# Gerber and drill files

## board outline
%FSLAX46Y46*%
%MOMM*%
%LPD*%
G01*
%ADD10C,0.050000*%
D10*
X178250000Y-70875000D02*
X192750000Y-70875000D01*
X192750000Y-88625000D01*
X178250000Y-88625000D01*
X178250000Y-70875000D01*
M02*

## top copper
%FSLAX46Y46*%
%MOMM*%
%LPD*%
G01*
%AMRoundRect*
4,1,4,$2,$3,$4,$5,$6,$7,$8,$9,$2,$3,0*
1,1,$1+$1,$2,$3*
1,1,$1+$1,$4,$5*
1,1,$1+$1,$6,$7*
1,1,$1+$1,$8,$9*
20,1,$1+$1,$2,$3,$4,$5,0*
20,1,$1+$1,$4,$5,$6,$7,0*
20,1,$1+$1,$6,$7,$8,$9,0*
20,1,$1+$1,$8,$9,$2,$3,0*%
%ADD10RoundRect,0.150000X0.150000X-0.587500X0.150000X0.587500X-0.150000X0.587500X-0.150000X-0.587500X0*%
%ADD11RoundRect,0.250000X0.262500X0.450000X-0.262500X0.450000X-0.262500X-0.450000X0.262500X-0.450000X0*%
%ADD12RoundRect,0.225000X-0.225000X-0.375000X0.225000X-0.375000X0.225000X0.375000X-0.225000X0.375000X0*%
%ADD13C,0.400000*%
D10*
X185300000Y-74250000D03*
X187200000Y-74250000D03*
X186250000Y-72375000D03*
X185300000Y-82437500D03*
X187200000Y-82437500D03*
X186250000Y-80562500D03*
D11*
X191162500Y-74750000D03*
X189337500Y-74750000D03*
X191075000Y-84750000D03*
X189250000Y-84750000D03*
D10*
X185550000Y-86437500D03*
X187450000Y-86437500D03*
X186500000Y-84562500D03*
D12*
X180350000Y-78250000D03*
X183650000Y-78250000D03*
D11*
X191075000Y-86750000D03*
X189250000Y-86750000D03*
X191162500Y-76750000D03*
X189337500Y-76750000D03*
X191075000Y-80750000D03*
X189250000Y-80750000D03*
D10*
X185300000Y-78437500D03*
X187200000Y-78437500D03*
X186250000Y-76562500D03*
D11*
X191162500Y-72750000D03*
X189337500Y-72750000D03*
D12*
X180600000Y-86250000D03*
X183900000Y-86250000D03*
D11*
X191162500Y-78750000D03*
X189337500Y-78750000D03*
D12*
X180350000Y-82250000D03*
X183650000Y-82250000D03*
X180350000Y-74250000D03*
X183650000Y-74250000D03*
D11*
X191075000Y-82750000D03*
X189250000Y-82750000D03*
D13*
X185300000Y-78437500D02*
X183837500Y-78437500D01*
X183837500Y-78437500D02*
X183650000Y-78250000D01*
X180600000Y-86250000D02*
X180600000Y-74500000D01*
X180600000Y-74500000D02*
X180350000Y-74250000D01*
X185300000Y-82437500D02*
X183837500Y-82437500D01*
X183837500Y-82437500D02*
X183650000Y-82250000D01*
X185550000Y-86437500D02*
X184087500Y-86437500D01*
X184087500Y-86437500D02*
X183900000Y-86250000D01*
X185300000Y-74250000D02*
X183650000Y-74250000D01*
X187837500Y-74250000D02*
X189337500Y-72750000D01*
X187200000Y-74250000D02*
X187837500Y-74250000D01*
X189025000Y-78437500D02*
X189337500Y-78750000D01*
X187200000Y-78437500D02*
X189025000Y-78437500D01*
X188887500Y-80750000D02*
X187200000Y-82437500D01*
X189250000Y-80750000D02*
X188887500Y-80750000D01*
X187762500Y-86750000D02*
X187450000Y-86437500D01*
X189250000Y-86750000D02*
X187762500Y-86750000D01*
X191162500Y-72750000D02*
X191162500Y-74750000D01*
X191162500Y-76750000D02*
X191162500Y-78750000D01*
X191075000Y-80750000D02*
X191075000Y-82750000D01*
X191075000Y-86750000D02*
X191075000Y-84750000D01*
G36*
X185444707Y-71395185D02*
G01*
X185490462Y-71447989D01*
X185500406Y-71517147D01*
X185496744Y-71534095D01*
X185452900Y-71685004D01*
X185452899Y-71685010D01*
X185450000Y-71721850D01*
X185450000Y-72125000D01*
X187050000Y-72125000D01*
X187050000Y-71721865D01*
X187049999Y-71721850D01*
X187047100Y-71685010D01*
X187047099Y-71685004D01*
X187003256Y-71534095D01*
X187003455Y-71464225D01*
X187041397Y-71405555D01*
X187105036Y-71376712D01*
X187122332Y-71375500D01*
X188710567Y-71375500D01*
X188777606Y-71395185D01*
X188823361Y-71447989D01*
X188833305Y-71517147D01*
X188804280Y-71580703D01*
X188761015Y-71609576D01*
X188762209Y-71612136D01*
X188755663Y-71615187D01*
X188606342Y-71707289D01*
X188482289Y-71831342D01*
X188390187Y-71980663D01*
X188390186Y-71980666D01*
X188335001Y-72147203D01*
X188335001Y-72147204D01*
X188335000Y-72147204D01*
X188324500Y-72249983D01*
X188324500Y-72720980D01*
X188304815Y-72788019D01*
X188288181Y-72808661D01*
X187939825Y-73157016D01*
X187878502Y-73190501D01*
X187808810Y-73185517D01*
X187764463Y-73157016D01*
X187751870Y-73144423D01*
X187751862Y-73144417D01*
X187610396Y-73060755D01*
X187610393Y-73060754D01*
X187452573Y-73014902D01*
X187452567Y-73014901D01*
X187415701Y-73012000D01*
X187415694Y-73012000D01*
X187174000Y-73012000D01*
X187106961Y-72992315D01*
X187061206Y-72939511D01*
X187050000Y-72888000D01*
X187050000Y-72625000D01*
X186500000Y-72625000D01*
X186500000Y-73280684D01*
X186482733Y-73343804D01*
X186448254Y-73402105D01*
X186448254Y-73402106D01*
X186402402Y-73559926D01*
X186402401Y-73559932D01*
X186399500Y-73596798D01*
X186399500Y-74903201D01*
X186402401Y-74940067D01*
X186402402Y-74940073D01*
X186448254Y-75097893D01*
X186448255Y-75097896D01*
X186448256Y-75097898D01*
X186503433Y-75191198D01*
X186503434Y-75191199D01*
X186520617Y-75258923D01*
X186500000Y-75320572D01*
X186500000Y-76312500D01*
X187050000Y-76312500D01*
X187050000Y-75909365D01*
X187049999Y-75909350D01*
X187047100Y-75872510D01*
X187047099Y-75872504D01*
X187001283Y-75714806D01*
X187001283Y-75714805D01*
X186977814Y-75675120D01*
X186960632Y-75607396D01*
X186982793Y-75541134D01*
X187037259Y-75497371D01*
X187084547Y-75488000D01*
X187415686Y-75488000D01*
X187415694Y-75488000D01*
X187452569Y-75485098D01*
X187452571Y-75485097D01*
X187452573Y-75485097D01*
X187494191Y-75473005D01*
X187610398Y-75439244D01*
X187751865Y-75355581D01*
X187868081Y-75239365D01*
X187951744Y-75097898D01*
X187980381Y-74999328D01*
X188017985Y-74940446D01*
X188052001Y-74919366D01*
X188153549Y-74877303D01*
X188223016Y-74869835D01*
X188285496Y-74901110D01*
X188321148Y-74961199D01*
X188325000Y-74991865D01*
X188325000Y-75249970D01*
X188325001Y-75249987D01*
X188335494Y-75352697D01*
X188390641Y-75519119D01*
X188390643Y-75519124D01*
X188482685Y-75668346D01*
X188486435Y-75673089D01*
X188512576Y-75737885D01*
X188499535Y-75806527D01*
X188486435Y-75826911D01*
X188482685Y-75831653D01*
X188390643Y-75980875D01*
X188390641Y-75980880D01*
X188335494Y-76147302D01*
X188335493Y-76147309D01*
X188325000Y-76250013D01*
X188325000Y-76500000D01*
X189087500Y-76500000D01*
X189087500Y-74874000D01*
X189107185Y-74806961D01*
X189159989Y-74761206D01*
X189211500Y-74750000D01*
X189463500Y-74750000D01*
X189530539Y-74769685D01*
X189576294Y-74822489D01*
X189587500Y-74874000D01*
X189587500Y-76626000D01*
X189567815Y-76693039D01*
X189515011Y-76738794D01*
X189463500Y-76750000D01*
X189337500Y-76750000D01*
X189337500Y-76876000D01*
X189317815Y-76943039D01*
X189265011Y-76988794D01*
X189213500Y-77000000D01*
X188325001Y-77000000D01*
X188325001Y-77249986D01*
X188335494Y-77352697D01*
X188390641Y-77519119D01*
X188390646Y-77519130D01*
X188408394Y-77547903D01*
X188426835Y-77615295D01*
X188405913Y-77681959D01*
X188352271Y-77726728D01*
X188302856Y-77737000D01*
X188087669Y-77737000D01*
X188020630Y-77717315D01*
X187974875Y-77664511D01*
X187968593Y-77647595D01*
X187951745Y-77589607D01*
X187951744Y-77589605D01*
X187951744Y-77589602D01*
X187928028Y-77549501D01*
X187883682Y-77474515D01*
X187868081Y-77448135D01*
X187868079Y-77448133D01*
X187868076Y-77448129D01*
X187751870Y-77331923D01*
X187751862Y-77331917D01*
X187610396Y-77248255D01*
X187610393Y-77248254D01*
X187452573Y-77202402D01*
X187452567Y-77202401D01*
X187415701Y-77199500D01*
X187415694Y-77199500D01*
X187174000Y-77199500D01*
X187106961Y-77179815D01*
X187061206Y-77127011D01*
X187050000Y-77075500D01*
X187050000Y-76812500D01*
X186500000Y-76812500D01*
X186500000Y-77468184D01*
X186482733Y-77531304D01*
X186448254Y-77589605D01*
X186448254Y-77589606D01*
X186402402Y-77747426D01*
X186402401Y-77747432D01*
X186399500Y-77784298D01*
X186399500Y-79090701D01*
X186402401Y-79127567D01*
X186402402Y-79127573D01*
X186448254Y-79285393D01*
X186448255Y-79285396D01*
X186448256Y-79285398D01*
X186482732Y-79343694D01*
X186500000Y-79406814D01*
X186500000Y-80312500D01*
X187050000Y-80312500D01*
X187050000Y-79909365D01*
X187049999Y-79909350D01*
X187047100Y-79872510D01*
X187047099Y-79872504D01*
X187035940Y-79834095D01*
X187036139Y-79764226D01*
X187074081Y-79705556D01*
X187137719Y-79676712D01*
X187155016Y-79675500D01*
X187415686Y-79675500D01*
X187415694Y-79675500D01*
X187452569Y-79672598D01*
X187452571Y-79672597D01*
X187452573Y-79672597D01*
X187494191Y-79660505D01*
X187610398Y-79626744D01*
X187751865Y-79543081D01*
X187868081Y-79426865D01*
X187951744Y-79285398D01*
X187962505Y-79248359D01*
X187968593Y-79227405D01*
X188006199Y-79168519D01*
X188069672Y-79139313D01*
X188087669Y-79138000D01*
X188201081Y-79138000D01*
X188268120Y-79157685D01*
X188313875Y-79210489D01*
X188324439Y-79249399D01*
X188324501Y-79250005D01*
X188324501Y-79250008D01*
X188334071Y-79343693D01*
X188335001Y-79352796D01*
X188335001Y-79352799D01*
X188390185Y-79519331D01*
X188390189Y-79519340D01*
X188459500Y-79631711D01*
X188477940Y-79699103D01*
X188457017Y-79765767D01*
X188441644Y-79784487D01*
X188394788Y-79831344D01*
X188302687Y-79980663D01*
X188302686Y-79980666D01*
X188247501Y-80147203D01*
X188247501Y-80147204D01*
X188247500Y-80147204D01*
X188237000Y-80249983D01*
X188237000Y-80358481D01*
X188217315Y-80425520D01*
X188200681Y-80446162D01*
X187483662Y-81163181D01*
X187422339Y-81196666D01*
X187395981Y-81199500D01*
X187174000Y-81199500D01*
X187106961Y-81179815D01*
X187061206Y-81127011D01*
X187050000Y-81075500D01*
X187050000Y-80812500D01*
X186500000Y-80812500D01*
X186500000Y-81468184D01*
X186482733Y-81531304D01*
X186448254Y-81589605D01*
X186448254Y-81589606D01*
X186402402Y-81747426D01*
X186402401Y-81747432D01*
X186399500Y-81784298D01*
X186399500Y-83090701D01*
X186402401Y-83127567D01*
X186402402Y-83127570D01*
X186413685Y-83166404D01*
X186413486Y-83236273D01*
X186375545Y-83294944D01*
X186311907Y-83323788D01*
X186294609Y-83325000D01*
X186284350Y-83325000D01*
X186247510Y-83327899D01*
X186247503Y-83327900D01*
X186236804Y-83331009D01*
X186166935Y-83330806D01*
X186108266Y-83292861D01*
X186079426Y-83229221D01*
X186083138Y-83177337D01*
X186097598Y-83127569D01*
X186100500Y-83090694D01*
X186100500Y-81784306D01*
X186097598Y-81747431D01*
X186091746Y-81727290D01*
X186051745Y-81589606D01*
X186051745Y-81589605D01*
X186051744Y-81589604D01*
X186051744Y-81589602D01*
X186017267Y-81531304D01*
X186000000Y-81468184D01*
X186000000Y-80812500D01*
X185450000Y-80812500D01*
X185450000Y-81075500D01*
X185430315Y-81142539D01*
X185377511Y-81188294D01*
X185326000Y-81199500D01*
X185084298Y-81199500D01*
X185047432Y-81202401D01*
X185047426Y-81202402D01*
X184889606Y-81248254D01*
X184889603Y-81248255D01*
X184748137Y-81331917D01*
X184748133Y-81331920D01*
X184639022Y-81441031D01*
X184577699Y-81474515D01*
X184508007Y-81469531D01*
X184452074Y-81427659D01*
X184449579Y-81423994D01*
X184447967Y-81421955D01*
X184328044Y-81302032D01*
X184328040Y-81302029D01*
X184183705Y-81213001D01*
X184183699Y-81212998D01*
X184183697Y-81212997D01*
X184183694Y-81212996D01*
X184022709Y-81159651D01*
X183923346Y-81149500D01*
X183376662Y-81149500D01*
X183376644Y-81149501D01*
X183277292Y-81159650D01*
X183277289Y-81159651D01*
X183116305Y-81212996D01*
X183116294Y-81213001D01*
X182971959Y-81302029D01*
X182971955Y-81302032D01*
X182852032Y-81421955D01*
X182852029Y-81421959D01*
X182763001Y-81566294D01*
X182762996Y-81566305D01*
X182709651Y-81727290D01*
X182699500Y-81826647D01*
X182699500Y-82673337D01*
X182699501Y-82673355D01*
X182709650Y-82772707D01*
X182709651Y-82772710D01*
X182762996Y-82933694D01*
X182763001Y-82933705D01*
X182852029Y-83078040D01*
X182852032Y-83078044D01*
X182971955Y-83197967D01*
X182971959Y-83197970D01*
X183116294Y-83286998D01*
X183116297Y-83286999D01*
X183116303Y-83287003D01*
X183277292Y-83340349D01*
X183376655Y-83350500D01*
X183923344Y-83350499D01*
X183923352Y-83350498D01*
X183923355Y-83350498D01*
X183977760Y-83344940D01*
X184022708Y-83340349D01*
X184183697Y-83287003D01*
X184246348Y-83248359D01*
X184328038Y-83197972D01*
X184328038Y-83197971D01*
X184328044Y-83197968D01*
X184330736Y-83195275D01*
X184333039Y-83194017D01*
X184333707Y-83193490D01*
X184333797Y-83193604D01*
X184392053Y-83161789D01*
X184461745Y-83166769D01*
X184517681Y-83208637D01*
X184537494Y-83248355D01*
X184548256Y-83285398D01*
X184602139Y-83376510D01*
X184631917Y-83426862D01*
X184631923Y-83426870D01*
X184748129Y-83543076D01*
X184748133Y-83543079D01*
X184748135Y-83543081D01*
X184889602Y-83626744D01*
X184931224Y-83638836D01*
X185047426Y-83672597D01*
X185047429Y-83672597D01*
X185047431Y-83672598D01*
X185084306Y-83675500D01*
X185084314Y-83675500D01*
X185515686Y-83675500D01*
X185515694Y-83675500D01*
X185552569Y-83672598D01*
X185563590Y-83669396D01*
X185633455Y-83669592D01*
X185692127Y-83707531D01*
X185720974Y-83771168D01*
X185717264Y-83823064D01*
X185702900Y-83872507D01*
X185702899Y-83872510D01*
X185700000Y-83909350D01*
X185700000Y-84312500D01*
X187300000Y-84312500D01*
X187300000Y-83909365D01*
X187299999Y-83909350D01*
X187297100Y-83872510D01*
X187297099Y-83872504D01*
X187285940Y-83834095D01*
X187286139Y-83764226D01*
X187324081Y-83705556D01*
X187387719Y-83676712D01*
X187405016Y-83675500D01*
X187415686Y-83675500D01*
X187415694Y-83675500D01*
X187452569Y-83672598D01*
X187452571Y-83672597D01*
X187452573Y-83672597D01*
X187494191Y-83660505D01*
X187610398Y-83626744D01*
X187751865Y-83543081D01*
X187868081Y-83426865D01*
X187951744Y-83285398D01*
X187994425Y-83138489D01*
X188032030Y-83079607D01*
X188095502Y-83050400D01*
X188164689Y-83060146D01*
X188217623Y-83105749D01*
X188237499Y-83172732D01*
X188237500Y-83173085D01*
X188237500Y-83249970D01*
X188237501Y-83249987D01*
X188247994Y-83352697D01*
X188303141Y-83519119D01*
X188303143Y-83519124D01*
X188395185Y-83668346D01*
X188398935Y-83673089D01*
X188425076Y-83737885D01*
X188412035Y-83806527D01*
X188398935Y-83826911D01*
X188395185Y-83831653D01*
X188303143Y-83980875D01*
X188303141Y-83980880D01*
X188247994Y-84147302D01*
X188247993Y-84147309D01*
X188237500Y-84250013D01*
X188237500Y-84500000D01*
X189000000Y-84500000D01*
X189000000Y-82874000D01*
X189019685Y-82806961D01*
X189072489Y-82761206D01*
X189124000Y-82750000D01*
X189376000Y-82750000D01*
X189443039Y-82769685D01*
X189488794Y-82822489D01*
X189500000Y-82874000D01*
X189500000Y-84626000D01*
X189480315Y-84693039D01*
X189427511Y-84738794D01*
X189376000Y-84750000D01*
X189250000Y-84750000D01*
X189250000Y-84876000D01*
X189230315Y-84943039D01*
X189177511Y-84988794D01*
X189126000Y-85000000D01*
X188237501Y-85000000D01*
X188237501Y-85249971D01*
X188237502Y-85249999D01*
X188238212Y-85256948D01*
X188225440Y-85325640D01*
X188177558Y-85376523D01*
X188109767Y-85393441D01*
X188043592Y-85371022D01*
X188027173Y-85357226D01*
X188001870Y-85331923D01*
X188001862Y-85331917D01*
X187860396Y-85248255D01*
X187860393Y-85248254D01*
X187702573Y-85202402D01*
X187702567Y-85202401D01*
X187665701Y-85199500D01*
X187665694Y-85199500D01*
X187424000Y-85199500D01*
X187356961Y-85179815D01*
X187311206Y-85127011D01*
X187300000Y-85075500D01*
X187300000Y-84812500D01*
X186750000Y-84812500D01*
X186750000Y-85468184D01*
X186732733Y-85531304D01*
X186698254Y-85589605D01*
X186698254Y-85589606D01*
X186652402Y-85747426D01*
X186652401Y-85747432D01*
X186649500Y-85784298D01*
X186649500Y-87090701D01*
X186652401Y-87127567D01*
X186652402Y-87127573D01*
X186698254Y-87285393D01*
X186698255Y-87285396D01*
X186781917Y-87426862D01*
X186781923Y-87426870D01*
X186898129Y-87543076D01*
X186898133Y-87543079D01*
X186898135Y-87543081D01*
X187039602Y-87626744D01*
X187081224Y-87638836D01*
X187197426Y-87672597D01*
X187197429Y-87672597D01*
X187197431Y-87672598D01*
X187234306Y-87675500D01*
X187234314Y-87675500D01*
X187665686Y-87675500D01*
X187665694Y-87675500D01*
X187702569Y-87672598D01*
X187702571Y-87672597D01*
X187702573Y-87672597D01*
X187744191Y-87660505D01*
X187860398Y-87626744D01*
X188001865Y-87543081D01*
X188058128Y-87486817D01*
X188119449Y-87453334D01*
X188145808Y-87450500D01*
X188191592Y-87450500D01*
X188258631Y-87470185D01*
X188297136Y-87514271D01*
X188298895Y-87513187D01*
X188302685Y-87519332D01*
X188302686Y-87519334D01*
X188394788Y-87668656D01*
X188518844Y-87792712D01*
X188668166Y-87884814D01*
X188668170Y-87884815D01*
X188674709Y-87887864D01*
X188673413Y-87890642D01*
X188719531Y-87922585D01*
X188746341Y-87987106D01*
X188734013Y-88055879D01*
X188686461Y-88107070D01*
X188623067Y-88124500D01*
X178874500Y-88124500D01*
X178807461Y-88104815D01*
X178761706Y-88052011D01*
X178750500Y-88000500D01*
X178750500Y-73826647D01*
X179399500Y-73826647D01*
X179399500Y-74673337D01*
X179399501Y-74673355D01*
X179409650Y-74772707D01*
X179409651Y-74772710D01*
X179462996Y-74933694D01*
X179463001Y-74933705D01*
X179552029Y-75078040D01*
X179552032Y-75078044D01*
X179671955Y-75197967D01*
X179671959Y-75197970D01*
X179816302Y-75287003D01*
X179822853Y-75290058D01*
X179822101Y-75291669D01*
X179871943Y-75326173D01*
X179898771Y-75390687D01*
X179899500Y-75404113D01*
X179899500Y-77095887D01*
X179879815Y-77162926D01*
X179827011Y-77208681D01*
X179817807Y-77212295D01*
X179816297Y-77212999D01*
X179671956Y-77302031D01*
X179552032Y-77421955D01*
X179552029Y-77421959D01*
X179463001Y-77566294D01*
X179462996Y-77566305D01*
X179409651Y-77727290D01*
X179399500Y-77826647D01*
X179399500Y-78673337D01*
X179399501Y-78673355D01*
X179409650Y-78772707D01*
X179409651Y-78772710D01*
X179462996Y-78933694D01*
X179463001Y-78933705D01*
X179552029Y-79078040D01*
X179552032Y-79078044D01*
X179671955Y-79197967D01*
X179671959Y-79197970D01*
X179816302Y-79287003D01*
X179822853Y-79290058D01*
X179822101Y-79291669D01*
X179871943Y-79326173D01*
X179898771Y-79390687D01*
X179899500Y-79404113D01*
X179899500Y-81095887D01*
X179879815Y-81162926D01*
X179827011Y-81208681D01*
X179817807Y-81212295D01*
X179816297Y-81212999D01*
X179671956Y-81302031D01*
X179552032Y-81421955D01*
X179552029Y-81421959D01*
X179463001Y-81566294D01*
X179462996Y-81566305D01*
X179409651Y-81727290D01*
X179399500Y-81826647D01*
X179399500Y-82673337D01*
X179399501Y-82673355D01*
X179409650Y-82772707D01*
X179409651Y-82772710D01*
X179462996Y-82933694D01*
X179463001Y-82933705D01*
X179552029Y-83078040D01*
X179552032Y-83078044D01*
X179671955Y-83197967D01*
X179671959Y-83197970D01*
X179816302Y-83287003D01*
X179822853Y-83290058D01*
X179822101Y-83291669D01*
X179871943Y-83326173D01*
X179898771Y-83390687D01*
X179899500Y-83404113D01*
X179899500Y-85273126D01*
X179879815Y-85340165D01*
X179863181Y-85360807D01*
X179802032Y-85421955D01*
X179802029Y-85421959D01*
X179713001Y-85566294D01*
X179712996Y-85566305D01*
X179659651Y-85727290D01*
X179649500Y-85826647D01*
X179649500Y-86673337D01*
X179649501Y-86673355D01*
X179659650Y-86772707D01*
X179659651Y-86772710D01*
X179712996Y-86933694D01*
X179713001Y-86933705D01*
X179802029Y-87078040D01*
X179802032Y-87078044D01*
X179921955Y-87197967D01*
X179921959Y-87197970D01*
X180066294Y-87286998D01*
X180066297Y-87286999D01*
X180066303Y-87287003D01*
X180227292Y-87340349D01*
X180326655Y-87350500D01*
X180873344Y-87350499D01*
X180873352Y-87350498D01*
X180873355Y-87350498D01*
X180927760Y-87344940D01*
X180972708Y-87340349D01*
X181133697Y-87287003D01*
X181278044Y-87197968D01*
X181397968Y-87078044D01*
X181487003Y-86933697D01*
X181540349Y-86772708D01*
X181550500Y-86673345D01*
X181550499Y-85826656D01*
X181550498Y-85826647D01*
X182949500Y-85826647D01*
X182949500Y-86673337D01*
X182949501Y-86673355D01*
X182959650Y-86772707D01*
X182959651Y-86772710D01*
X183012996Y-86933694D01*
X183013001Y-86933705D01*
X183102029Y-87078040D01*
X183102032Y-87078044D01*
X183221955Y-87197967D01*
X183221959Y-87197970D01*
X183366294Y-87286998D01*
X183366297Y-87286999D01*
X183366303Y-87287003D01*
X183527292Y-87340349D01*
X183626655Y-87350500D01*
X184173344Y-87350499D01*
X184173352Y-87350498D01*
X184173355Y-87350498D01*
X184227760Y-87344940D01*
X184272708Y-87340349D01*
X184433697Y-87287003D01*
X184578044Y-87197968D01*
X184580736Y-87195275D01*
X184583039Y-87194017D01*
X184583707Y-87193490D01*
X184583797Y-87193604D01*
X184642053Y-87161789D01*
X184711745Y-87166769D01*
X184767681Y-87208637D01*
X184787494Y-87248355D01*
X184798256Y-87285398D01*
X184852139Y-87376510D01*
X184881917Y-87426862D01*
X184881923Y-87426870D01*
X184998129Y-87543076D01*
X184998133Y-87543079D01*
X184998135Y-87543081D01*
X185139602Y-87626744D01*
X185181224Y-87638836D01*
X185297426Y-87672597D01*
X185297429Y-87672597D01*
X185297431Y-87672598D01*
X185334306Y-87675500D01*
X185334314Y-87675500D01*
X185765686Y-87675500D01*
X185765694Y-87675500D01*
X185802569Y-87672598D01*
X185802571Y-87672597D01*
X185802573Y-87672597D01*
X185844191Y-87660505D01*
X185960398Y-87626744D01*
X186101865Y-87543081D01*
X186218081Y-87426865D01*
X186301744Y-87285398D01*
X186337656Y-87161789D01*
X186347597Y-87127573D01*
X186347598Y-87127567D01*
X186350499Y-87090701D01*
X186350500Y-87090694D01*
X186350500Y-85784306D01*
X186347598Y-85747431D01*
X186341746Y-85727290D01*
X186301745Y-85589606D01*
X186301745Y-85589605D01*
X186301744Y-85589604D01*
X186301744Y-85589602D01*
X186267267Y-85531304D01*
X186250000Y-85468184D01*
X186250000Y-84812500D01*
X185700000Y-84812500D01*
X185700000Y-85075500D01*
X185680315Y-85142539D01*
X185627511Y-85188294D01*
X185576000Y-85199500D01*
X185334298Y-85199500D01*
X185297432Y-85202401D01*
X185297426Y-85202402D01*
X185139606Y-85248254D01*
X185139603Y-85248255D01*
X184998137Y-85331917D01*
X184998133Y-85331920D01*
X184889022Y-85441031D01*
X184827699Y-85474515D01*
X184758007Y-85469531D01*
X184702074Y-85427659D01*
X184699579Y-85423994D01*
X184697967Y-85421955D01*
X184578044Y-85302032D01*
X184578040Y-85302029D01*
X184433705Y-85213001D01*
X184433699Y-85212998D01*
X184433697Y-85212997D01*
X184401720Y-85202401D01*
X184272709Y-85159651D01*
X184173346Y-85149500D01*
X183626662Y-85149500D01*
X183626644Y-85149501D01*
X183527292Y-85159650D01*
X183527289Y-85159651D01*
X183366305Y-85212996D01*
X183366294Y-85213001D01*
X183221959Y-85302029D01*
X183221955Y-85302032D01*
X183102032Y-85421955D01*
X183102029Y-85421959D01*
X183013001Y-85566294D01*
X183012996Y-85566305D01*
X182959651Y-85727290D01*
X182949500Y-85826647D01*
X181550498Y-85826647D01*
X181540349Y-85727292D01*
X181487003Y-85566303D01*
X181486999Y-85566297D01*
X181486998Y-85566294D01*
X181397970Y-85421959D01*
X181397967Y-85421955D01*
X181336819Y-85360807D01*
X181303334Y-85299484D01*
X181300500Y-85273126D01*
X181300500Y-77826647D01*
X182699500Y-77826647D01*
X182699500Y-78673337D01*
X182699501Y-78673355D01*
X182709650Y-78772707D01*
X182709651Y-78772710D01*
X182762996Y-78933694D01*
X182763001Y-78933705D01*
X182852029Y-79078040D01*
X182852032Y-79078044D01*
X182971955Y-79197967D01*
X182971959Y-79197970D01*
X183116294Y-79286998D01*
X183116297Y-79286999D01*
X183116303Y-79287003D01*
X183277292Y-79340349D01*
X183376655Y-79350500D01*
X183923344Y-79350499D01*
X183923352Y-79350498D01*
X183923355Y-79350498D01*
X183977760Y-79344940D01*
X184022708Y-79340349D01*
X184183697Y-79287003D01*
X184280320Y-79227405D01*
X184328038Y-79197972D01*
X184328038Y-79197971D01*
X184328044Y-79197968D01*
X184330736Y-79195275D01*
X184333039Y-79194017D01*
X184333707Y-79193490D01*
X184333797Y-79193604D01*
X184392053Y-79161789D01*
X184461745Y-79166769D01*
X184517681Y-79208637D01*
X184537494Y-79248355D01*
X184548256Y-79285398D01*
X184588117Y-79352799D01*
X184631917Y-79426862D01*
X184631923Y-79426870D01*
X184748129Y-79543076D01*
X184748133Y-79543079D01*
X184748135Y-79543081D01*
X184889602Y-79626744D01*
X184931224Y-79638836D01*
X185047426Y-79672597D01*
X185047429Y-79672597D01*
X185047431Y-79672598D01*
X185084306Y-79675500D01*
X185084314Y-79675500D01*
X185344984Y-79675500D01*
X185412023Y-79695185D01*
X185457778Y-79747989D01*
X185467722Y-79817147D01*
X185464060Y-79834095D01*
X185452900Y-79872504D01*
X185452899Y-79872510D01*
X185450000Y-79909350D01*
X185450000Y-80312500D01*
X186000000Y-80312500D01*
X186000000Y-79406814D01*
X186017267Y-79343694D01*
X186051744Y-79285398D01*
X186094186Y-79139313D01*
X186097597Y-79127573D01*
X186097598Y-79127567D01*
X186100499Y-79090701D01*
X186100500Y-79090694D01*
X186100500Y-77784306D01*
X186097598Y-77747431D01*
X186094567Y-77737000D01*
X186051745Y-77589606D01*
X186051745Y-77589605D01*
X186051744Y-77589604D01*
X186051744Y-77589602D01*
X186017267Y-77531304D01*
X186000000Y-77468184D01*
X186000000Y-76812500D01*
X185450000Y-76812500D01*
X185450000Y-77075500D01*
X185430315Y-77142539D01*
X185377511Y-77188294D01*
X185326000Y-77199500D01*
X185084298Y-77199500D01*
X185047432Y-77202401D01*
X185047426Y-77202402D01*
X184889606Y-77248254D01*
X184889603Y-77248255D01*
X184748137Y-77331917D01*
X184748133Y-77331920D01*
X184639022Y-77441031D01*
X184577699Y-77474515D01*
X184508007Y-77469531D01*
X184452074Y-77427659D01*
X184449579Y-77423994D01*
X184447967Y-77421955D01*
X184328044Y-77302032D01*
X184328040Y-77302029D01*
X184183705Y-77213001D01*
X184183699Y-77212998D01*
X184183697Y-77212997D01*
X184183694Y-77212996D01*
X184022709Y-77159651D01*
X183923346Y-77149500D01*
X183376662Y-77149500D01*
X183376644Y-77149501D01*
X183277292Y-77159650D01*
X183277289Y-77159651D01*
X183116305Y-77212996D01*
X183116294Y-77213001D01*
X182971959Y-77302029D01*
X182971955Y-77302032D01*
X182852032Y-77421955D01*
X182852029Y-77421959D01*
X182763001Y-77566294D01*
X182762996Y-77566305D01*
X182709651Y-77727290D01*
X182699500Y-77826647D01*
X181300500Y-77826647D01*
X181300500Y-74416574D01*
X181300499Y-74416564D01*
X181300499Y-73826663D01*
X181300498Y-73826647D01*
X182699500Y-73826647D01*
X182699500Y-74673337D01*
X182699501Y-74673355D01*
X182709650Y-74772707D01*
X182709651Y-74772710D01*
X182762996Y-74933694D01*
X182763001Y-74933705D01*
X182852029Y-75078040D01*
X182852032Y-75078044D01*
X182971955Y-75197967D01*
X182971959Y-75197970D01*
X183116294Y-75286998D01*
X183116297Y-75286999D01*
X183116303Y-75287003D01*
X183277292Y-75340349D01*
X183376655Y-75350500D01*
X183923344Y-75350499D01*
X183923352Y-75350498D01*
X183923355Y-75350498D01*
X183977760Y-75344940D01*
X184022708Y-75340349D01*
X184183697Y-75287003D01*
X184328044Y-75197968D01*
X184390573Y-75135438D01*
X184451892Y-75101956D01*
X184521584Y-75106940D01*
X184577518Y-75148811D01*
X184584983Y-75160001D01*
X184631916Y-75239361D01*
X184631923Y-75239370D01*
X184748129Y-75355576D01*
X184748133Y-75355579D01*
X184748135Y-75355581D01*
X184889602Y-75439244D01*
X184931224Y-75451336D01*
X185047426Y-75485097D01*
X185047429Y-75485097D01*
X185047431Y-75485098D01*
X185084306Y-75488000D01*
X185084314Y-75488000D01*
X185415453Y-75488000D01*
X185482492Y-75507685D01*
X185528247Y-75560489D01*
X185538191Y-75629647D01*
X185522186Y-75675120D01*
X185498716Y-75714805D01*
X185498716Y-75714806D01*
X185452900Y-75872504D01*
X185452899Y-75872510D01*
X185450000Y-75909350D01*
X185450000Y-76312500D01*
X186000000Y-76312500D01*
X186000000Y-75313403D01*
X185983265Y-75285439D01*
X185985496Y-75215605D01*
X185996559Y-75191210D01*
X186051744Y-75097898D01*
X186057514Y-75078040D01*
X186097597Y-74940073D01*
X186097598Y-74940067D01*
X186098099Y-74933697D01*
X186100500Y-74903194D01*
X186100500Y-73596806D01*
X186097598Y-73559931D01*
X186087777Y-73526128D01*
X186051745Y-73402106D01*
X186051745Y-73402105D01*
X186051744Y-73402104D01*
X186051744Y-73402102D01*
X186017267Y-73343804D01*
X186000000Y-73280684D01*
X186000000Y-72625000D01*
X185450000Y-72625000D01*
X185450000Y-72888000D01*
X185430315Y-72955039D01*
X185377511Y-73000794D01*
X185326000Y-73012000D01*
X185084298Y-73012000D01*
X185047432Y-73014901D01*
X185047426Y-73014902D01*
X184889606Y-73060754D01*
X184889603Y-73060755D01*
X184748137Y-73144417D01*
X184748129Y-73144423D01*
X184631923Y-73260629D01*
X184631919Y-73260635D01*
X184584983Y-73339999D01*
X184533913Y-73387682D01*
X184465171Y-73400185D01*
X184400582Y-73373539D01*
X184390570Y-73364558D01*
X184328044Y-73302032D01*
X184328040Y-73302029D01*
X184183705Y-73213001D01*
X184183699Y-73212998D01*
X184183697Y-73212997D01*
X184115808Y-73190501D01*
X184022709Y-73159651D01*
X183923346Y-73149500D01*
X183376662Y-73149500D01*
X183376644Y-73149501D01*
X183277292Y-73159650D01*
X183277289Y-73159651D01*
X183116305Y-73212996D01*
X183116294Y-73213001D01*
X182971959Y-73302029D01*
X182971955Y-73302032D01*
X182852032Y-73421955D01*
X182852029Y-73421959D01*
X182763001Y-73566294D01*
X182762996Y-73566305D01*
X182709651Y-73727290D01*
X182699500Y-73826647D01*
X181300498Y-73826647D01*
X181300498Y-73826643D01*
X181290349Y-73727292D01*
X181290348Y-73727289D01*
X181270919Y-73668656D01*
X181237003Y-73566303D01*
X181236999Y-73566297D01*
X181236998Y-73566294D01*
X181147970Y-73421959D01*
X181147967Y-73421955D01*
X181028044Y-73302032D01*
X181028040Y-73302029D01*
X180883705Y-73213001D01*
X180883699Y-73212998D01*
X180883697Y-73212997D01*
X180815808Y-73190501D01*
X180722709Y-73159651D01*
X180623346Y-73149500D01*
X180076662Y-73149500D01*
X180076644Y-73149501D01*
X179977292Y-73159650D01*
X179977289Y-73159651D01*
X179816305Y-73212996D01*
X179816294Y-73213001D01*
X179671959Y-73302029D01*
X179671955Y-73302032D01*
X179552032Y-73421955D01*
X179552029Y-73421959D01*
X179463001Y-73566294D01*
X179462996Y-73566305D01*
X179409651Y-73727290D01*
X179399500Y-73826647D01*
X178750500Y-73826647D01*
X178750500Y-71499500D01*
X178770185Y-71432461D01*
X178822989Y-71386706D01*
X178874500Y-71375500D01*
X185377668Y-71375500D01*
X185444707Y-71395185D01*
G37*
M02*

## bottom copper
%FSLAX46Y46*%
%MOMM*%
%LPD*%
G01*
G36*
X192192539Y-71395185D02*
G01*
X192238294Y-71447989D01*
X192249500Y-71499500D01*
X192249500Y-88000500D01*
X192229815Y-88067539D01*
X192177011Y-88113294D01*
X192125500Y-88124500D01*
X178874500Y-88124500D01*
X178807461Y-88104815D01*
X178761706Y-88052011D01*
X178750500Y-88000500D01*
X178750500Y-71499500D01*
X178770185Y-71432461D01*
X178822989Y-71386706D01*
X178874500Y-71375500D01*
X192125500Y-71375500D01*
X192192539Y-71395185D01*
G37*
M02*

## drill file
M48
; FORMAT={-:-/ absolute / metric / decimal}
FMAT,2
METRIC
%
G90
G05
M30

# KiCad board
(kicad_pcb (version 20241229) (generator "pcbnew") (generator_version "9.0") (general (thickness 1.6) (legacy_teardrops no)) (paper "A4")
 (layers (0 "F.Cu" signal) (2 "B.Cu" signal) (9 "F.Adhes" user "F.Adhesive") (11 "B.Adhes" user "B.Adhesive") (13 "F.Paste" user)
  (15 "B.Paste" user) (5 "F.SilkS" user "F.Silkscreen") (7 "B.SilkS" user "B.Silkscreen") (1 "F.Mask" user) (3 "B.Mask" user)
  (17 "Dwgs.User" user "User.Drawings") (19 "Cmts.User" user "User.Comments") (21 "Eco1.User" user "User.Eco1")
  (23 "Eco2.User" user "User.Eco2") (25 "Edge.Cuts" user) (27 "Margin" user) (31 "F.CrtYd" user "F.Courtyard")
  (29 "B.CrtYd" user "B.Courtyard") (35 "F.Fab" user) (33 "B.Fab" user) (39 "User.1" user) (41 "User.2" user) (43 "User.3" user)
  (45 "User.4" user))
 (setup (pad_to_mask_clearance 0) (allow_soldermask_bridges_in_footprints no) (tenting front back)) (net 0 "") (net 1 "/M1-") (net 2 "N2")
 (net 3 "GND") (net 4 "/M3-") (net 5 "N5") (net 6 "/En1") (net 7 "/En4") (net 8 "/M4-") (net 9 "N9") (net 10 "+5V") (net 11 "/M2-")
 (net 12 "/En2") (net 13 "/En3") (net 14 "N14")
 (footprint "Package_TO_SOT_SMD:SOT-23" (layer "F.Cu") (at 186.25 73.3125 90)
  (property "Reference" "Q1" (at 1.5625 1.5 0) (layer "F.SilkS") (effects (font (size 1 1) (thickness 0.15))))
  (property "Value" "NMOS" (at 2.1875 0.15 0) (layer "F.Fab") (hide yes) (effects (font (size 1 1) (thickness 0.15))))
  (pad "1" smd roundrect (at -0.9375 -0.95 90) (size 1.475 0.6) (layers "F.Cu" "F.Mask" "F.Paste") (roundrect_rratio 0.25) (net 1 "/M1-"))
  (pad "2" smd roundrect (at -0.9375 0.95 90) (size 1.475 0.6) (layers "F.Cu" "F.Mask" "F.Paste") (roundrect_rratio 0.25) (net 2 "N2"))
  (pad "3" smd roundrect (at 0.9375 0 90) (size 1.475 0.6) (layers "F.Cu" "F.Mask" "F.Paste") (roundrect_rratio 0.25) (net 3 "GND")))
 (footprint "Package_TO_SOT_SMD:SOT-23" (layer "F.Cu") (at 186.25 81.5 90)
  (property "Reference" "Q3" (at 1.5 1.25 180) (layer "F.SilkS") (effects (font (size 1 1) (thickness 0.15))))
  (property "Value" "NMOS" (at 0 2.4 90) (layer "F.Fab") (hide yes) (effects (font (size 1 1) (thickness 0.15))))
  (pad "1" smd roundrect (at -0.9375 -0.95 90) (size 1.475 0.6) (layers "F.Cu" "F.Mask" "F.Paste") (roundrect_rratio 0.25) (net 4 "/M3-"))
  (pad "2" smd roundrect (at -0.9375 0.95 90) (size 1.475 0.6) (layers "F.Cu" "F.Mask" "F.Paste") (roundrect_rratio 0.25) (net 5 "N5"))
  (pad "3" smd roundrect (at 0.9375 0 90) (size 1.475 0.6) (layers "F.Cu" "F.Mask" "F.Paste") (roundrect_rratio 0.25) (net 3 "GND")))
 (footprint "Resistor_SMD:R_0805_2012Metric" (layer "F.Cu") (at 190.25 74.75 180)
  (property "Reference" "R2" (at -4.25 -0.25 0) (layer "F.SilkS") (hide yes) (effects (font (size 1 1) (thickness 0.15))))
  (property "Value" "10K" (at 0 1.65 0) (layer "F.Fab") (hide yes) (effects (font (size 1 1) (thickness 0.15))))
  (pad "1" smd roundrect (at -0.9125 0 180) (size 1.025 1.4) (layers "F.Cu" "F.Mask" "F.Paste") (roundrect_rratio 0.243902) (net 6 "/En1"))
  (pad "2" smd roundrect (at 0.9125 0 180) (size 1.025 1.4) (layers "F.Cu" "F.Mask" "F.Paste") (roundrect_rratio 0.243902) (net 3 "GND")))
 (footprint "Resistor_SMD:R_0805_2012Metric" (layer "F.Cu") (at 190.1625 84.75 180)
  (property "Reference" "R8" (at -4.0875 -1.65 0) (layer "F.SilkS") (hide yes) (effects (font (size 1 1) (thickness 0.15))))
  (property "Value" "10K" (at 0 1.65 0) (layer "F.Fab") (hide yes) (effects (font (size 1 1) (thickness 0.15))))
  (pad "1" smd roundrect (at -0.9125 0 180) (size 1.025 1.4) (layers "F.Cu" "F.Mask" "F.Paste") (roundrect_rratio 0.243902) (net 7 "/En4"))
  (pad "2" smd roundrect (at 0.9125 0 180) (size 1.025 1.4) (layers "F.Cu" "F.Mask" "F.Paste") (roundrect_rratio 0.243902) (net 3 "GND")))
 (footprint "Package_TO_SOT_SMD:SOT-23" (layer "F.Cu") (at 186.5 85.5 90)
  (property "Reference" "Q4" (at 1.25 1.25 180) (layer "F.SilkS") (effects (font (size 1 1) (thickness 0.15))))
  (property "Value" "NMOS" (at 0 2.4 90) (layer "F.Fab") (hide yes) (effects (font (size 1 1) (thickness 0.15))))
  (pad "1" smd roundrect (at -0.9375 -0.95 90) (size 1.475 0.6) (layers "F.Cu" "F.Mask" "F.Paste") (roundrect_rratio 0.25) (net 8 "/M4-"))
  (pad "2" smd roundrect (at -0.9375 0.95 90) (size 1.475 0.6) (layers "F.Cu" "F.Mask" "F.Paste") (roundrect_rratio 0.25) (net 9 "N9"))
  (pad "3" smd roundrect (at 0.9375 0 90) (size 1.475 0.6) (layers "F.Cu" "F.Mask" "F.Paste") (roundrect_rratio 0.25) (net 3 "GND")))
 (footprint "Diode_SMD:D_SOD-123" (layer "F.Cu") (at 182 78.25)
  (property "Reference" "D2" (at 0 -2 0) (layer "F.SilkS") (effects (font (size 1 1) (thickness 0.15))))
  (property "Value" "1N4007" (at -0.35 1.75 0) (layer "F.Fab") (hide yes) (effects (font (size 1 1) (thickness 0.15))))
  (pad "1" smd roundrect (at -1.65 0) (size 0.9 1.2) (layers "F.Cu" "F.Mask" "F.Paste") (roundrect_rratio 0.25) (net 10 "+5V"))
  (pad "2" smd roundrect (at 1.65 0) (size 0.9 1.2) (layers "F.Cu" "F.Mask" "F.Paste") (roundrect_rratio 0.25) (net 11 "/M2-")))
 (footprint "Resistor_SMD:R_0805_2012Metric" (layer "F.Cu") (at 190.1625 86.75 180)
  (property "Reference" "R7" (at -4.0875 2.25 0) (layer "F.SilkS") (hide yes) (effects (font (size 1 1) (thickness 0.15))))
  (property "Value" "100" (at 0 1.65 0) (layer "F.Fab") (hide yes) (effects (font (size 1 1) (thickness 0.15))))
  (pad "1" smd roundrect (at -0.9125 0 180) (size 1.025 1.4) (layers "F.Cu" "F.Mask" "F.Paste") (roundrect_rratio 0.243902) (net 7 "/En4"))
  (pad "2" smd roundrect (at 0.9125 0 180) (size 1.025 1.4) (layers "F.Cu" "F.Mask" "F.Paste") (roundrect_rratio 0.243902) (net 9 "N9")))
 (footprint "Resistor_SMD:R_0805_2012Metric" (layer "F.Cu") (at 190.25 76.75 180)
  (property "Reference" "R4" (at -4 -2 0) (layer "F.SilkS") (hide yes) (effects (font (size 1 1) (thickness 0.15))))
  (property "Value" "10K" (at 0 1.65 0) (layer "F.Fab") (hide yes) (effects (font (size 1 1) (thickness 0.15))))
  (pad "1" smd roundrect (at -0.9125 0 180) (size 1.025 1.4) (layers "F.Cu" "F.Mask" "F.Paste") (roundrect_rratio 0.243902) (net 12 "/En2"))
  (pad "2" smd roundrect (at 0.9125 0 180) (size 1.025 1.4) (layers "F.Cu" "F.Mask" "F.Paste") (roundrect_rratio 0.243902) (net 3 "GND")))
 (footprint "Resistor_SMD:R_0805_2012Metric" (layer "F.Cu") (at 190.1625 80.75 180)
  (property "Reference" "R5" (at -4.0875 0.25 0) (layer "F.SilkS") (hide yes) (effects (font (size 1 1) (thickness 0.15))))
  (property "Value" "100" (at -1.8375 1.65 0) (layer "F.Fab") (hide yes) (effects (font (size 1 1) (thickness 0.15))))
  (pad "1" smd roundrect (at -0.9125 0 180) (size 1.025 1.4) (layers "F.Cu" "F.Mask" "F.Paste") (roundrect_rratio 0.243902) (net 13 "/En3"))
  (pad "2" smd roundrect (at 0.9125 0 180) (size 1.025 1.4) (layers "F.Cu" "F.Mask" "F.Paste") (roundrect_rratio 0.243902) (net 5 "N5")))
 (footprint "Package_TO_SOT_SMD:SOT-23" (layer "F.Cu") (at 186.25 77.5 90)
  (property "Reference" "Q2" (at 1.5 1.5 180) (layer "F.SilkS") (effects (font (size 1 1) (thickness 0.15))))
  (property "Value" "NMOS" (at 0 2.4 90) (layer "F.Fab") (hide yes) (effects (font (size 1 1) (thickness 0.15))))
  (pad "1" smd roundrect (at -0.9375 -0.95 90) (size 1.475 0.6) (layers "F.Cu" "F.Mask" "F.Paste") (roundrect_rratio 0.25) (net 11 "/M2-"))
  (pad "2" smd roundrect (at -0.9375 0.95 90) (size 1.475 0.6) (layers "F.Cu" "F.Mask" "F.Paste") (roundrect_rratio 0.25) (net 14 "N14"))
  (pad "3" smd roundrect (at 0.9375 0 90) (size 1.475 0.6) (layers "F.Cu" "F.Mask" "F.Paste") (roundrect_rratio 0.25) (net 3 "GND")))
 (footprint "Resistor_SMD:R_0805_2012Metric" (layer "F.Cu") (at 190.25 72.75 180)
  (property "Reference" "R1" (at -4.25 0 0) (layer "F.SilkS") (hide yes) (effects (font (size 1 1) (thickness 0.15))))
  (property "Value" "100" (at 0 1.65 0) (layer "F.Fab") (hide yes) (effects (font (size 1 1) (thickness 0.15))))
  (pad "1" smd roundrect (at -0.9125 0 180) (size 1.025 1.4) (layers "F.Cu" "F.Mask" "F.Paste") (roundrect_rratio 0.243902) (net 6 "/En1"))
  (pad "2" smd roundrect (at 0.9125 0 180) (size 1.025 1.4) (layers "F.Cu" "F.Mask" "F.Paste") (roundrect_rratio 0.243902) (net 2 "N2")))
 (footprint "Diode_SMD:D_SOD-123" (layer "F.Cu") (at 182.25 86.25)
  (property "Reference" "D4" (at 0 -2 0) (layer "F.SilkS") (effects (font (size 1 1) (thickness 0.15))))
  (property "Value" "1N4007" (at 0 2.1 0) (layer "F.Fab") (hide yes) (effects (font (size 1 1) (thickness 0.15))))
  (pad "1" smd roundrect (at -1.65 0) (size 0.9 1.2) (layers "F.Cu" "F.Mask" "F.Paste") (roundrect_rratio 0.25) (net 10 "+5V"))
  (pad "2" smd roundrect (at 1.65 0) (size 0.9 1.2) (layers "F.Cu" "F.Mask" "F.Paste") (roundrect_rratio 0.25) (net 8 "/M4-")))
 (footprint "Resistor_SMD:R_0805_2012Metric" (layer "F.Cu") (at 190.25 78.75 180)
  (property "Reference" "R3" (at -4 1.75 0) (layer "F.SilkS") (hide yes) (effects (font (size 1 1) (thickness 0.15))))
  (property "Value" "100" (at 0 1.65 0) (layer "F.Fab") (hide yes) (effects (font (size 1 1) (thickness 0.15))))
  (pad "1" smd roundrect (at -0.9125 0 180) (size 1.025 1.4) (layers "F.Cu" "F.Mask" "F.Paste") (roundrect_rratio 0.243902) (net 12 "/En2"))
  (pad "2" smd roundrect (at 0.9125 0 180) (size 1.025 1.4) (layers "F.Cu" "F.Mask" "F.Paste") (roundrect_rratio 0.243902) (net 14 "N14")))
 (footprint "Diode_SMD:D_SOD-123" (layer "F.Cu") (at 182 82.25)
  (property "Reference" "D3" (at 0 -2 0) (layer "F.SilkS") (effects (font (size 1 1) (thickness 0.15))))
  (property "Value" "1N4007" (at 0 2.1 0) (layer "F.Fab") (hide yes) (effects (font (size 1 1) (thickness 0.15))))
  (pad "1" smd roundrect (at -1.65 0) (size 0.9 1.2) (layers "F.Cu" "F.Mask" "F.Paste") (roundrect_rratio 0.25) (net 10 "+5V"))
  (pad "2" smd roundrect (at 1.65 0) (size 0.9 1.2) (layers "F.Cu" "F.Mask" "F.Paste") (roundrect_rratio 0.25) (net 4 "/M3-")))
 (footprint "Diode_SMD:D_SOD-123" (layer "F.Cu") (at 182 74.25)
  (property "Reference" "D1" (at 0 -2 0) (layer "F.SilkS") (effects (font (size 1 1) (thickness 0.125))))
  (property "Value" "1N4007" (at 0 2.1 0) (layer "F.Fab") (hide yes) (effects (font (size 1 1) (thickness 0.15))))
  (pad "1" smd roundrect (at -1.65 0) (size 0.9 1.2) (layers "F.Cu" "F.Mask" "F.Paste") (roundrect_rratio 0.25) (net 10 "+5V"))
  (pad "2" smd roundrect (at 1.65 0) (size 0.9 1.2) (layers "F.Cu" "F.Mask" "F.Paste") (roundrect_rratio 0.25) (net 1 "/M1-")))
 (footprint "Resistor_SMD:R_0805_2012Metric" (layer "F.Cu") (at 190.1625 82.75 180)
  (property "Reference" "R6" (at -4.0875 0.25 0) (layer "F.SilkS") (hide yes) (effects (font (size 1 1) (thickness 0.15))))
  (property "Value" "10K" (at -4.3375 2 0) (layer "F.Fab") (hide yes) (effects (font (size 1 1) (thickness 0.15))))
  (pad "1" smd roundrect (at -0.9125 0 180) (size 1.025 1.4) (layers "F.Cu" "F.Mask" "F.Paste") (roundrect_rratio 0.243902) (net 13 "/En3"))
  (pad "2" smd roundrect (at 0.9125 0 180) (size 1.025 1.4) (layers "F.Cu" "F.Mask" "F.Paste") (roundrect_rratio 0.243902) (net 3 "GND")))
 (gr_rect (start 178.25 70.875) (end 192.75 88.625) (stroke (width 0.05) (type default)) (fill no) (layer "Edge.Cuts"))
 (segment (start 185.3 78.4375) (end 183.8375 78.4375) (width 0.4) (layer "F.Cu") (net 11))
 (segment (start 183.8375 78.4375) (end 183.65 78.25) (width 0.4) (layer "F.Cu") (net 11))
 (segment (start 180.6 86.25) (end 180.6 74.5) (width 0.4) (layer "F.Cu") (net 10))
 (segment (start 180.6 74.5) (end 180.35 74.25) (width 0.4) (layer "F.Cu") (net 10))
 (segment (start 185.3 82.4375) (end 183.8375 82.4375) (width 0.4) (layer "F.Cu") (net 4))
 (segment (start 183.8375 82.4375) (end 183.65 82.25) (width 0.4) (layer "F.Cu") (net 4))
 (segment (start 185.55 86.4375) (end 184.0875 86.4375) (width 0.4) (layer "F.Cu") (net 8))
 (segment (start 184.0875 86.4375) (end 183.9 86.25) (width 0.4) (layer "F.Cu") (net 8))
 (segment (start 185.3 74.25) (end 183.65 74.25) (width 0.4) (layer "F.Cu") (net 1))
 (segment (start 187.8375 74.25) (end 189.3375 72.75) (width 0.4) (layer "F.Cu") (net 2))
 (segment (start 187.2 74.25) (end 187.8375 74.25) (width 0.4) (layer "F.Cu") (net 2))
 (segment (start 189.025 78.4375) (end 189.3375 78.75) (width 0.4) (layer "F.Cu") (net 14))
 (segment (start 187.2 78.4375) (end 189.025 78.4375) (width 0.4) (layer "F.Cu") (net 14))
 (segment (start 188.8875 80.75) (end 187.2 82.4375) (width 0.4) (layer "F.Cu") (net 5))
 (segment (start 189.25 80.75) (end 188.8875 80.75) (width 0.4) (layer "F.Cu") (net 5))
 (segment (start 187.7625 86.75) (end 187.45 86.4375) (width 0.4) (layer "F.Cu") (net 9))
 (segment (start 189.25 86.75) (end 187.7625 86.75) (width 0.4) (layer "F.Cu") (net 9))
 (segment (start 191.1625 72.75) (end 191.1625 74.75) (width 0.4) (layer "F.Cu") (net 6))
 (segment (start 191.1625 76.75) (end 191.1625 78.75) (width 0.4) (layer "F.Cu") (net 12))
 (segment (start 191.075 80.75) (end 191.075 82.75) (width 0.4) (layer "F.Cu") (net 13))
 (segment (start 191.075 86.75) (end 191.075 84.75) (width 0.4) (layer "F.Cu") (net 7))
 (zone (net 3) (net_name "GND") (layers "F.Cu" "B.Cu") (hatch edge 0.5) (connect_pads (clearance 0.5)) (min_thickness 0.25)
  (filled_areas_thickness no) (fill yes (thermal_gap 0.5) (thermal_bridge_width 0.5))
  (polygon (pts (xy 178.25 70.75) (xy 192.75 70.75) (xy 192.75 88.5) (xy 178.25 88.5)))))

